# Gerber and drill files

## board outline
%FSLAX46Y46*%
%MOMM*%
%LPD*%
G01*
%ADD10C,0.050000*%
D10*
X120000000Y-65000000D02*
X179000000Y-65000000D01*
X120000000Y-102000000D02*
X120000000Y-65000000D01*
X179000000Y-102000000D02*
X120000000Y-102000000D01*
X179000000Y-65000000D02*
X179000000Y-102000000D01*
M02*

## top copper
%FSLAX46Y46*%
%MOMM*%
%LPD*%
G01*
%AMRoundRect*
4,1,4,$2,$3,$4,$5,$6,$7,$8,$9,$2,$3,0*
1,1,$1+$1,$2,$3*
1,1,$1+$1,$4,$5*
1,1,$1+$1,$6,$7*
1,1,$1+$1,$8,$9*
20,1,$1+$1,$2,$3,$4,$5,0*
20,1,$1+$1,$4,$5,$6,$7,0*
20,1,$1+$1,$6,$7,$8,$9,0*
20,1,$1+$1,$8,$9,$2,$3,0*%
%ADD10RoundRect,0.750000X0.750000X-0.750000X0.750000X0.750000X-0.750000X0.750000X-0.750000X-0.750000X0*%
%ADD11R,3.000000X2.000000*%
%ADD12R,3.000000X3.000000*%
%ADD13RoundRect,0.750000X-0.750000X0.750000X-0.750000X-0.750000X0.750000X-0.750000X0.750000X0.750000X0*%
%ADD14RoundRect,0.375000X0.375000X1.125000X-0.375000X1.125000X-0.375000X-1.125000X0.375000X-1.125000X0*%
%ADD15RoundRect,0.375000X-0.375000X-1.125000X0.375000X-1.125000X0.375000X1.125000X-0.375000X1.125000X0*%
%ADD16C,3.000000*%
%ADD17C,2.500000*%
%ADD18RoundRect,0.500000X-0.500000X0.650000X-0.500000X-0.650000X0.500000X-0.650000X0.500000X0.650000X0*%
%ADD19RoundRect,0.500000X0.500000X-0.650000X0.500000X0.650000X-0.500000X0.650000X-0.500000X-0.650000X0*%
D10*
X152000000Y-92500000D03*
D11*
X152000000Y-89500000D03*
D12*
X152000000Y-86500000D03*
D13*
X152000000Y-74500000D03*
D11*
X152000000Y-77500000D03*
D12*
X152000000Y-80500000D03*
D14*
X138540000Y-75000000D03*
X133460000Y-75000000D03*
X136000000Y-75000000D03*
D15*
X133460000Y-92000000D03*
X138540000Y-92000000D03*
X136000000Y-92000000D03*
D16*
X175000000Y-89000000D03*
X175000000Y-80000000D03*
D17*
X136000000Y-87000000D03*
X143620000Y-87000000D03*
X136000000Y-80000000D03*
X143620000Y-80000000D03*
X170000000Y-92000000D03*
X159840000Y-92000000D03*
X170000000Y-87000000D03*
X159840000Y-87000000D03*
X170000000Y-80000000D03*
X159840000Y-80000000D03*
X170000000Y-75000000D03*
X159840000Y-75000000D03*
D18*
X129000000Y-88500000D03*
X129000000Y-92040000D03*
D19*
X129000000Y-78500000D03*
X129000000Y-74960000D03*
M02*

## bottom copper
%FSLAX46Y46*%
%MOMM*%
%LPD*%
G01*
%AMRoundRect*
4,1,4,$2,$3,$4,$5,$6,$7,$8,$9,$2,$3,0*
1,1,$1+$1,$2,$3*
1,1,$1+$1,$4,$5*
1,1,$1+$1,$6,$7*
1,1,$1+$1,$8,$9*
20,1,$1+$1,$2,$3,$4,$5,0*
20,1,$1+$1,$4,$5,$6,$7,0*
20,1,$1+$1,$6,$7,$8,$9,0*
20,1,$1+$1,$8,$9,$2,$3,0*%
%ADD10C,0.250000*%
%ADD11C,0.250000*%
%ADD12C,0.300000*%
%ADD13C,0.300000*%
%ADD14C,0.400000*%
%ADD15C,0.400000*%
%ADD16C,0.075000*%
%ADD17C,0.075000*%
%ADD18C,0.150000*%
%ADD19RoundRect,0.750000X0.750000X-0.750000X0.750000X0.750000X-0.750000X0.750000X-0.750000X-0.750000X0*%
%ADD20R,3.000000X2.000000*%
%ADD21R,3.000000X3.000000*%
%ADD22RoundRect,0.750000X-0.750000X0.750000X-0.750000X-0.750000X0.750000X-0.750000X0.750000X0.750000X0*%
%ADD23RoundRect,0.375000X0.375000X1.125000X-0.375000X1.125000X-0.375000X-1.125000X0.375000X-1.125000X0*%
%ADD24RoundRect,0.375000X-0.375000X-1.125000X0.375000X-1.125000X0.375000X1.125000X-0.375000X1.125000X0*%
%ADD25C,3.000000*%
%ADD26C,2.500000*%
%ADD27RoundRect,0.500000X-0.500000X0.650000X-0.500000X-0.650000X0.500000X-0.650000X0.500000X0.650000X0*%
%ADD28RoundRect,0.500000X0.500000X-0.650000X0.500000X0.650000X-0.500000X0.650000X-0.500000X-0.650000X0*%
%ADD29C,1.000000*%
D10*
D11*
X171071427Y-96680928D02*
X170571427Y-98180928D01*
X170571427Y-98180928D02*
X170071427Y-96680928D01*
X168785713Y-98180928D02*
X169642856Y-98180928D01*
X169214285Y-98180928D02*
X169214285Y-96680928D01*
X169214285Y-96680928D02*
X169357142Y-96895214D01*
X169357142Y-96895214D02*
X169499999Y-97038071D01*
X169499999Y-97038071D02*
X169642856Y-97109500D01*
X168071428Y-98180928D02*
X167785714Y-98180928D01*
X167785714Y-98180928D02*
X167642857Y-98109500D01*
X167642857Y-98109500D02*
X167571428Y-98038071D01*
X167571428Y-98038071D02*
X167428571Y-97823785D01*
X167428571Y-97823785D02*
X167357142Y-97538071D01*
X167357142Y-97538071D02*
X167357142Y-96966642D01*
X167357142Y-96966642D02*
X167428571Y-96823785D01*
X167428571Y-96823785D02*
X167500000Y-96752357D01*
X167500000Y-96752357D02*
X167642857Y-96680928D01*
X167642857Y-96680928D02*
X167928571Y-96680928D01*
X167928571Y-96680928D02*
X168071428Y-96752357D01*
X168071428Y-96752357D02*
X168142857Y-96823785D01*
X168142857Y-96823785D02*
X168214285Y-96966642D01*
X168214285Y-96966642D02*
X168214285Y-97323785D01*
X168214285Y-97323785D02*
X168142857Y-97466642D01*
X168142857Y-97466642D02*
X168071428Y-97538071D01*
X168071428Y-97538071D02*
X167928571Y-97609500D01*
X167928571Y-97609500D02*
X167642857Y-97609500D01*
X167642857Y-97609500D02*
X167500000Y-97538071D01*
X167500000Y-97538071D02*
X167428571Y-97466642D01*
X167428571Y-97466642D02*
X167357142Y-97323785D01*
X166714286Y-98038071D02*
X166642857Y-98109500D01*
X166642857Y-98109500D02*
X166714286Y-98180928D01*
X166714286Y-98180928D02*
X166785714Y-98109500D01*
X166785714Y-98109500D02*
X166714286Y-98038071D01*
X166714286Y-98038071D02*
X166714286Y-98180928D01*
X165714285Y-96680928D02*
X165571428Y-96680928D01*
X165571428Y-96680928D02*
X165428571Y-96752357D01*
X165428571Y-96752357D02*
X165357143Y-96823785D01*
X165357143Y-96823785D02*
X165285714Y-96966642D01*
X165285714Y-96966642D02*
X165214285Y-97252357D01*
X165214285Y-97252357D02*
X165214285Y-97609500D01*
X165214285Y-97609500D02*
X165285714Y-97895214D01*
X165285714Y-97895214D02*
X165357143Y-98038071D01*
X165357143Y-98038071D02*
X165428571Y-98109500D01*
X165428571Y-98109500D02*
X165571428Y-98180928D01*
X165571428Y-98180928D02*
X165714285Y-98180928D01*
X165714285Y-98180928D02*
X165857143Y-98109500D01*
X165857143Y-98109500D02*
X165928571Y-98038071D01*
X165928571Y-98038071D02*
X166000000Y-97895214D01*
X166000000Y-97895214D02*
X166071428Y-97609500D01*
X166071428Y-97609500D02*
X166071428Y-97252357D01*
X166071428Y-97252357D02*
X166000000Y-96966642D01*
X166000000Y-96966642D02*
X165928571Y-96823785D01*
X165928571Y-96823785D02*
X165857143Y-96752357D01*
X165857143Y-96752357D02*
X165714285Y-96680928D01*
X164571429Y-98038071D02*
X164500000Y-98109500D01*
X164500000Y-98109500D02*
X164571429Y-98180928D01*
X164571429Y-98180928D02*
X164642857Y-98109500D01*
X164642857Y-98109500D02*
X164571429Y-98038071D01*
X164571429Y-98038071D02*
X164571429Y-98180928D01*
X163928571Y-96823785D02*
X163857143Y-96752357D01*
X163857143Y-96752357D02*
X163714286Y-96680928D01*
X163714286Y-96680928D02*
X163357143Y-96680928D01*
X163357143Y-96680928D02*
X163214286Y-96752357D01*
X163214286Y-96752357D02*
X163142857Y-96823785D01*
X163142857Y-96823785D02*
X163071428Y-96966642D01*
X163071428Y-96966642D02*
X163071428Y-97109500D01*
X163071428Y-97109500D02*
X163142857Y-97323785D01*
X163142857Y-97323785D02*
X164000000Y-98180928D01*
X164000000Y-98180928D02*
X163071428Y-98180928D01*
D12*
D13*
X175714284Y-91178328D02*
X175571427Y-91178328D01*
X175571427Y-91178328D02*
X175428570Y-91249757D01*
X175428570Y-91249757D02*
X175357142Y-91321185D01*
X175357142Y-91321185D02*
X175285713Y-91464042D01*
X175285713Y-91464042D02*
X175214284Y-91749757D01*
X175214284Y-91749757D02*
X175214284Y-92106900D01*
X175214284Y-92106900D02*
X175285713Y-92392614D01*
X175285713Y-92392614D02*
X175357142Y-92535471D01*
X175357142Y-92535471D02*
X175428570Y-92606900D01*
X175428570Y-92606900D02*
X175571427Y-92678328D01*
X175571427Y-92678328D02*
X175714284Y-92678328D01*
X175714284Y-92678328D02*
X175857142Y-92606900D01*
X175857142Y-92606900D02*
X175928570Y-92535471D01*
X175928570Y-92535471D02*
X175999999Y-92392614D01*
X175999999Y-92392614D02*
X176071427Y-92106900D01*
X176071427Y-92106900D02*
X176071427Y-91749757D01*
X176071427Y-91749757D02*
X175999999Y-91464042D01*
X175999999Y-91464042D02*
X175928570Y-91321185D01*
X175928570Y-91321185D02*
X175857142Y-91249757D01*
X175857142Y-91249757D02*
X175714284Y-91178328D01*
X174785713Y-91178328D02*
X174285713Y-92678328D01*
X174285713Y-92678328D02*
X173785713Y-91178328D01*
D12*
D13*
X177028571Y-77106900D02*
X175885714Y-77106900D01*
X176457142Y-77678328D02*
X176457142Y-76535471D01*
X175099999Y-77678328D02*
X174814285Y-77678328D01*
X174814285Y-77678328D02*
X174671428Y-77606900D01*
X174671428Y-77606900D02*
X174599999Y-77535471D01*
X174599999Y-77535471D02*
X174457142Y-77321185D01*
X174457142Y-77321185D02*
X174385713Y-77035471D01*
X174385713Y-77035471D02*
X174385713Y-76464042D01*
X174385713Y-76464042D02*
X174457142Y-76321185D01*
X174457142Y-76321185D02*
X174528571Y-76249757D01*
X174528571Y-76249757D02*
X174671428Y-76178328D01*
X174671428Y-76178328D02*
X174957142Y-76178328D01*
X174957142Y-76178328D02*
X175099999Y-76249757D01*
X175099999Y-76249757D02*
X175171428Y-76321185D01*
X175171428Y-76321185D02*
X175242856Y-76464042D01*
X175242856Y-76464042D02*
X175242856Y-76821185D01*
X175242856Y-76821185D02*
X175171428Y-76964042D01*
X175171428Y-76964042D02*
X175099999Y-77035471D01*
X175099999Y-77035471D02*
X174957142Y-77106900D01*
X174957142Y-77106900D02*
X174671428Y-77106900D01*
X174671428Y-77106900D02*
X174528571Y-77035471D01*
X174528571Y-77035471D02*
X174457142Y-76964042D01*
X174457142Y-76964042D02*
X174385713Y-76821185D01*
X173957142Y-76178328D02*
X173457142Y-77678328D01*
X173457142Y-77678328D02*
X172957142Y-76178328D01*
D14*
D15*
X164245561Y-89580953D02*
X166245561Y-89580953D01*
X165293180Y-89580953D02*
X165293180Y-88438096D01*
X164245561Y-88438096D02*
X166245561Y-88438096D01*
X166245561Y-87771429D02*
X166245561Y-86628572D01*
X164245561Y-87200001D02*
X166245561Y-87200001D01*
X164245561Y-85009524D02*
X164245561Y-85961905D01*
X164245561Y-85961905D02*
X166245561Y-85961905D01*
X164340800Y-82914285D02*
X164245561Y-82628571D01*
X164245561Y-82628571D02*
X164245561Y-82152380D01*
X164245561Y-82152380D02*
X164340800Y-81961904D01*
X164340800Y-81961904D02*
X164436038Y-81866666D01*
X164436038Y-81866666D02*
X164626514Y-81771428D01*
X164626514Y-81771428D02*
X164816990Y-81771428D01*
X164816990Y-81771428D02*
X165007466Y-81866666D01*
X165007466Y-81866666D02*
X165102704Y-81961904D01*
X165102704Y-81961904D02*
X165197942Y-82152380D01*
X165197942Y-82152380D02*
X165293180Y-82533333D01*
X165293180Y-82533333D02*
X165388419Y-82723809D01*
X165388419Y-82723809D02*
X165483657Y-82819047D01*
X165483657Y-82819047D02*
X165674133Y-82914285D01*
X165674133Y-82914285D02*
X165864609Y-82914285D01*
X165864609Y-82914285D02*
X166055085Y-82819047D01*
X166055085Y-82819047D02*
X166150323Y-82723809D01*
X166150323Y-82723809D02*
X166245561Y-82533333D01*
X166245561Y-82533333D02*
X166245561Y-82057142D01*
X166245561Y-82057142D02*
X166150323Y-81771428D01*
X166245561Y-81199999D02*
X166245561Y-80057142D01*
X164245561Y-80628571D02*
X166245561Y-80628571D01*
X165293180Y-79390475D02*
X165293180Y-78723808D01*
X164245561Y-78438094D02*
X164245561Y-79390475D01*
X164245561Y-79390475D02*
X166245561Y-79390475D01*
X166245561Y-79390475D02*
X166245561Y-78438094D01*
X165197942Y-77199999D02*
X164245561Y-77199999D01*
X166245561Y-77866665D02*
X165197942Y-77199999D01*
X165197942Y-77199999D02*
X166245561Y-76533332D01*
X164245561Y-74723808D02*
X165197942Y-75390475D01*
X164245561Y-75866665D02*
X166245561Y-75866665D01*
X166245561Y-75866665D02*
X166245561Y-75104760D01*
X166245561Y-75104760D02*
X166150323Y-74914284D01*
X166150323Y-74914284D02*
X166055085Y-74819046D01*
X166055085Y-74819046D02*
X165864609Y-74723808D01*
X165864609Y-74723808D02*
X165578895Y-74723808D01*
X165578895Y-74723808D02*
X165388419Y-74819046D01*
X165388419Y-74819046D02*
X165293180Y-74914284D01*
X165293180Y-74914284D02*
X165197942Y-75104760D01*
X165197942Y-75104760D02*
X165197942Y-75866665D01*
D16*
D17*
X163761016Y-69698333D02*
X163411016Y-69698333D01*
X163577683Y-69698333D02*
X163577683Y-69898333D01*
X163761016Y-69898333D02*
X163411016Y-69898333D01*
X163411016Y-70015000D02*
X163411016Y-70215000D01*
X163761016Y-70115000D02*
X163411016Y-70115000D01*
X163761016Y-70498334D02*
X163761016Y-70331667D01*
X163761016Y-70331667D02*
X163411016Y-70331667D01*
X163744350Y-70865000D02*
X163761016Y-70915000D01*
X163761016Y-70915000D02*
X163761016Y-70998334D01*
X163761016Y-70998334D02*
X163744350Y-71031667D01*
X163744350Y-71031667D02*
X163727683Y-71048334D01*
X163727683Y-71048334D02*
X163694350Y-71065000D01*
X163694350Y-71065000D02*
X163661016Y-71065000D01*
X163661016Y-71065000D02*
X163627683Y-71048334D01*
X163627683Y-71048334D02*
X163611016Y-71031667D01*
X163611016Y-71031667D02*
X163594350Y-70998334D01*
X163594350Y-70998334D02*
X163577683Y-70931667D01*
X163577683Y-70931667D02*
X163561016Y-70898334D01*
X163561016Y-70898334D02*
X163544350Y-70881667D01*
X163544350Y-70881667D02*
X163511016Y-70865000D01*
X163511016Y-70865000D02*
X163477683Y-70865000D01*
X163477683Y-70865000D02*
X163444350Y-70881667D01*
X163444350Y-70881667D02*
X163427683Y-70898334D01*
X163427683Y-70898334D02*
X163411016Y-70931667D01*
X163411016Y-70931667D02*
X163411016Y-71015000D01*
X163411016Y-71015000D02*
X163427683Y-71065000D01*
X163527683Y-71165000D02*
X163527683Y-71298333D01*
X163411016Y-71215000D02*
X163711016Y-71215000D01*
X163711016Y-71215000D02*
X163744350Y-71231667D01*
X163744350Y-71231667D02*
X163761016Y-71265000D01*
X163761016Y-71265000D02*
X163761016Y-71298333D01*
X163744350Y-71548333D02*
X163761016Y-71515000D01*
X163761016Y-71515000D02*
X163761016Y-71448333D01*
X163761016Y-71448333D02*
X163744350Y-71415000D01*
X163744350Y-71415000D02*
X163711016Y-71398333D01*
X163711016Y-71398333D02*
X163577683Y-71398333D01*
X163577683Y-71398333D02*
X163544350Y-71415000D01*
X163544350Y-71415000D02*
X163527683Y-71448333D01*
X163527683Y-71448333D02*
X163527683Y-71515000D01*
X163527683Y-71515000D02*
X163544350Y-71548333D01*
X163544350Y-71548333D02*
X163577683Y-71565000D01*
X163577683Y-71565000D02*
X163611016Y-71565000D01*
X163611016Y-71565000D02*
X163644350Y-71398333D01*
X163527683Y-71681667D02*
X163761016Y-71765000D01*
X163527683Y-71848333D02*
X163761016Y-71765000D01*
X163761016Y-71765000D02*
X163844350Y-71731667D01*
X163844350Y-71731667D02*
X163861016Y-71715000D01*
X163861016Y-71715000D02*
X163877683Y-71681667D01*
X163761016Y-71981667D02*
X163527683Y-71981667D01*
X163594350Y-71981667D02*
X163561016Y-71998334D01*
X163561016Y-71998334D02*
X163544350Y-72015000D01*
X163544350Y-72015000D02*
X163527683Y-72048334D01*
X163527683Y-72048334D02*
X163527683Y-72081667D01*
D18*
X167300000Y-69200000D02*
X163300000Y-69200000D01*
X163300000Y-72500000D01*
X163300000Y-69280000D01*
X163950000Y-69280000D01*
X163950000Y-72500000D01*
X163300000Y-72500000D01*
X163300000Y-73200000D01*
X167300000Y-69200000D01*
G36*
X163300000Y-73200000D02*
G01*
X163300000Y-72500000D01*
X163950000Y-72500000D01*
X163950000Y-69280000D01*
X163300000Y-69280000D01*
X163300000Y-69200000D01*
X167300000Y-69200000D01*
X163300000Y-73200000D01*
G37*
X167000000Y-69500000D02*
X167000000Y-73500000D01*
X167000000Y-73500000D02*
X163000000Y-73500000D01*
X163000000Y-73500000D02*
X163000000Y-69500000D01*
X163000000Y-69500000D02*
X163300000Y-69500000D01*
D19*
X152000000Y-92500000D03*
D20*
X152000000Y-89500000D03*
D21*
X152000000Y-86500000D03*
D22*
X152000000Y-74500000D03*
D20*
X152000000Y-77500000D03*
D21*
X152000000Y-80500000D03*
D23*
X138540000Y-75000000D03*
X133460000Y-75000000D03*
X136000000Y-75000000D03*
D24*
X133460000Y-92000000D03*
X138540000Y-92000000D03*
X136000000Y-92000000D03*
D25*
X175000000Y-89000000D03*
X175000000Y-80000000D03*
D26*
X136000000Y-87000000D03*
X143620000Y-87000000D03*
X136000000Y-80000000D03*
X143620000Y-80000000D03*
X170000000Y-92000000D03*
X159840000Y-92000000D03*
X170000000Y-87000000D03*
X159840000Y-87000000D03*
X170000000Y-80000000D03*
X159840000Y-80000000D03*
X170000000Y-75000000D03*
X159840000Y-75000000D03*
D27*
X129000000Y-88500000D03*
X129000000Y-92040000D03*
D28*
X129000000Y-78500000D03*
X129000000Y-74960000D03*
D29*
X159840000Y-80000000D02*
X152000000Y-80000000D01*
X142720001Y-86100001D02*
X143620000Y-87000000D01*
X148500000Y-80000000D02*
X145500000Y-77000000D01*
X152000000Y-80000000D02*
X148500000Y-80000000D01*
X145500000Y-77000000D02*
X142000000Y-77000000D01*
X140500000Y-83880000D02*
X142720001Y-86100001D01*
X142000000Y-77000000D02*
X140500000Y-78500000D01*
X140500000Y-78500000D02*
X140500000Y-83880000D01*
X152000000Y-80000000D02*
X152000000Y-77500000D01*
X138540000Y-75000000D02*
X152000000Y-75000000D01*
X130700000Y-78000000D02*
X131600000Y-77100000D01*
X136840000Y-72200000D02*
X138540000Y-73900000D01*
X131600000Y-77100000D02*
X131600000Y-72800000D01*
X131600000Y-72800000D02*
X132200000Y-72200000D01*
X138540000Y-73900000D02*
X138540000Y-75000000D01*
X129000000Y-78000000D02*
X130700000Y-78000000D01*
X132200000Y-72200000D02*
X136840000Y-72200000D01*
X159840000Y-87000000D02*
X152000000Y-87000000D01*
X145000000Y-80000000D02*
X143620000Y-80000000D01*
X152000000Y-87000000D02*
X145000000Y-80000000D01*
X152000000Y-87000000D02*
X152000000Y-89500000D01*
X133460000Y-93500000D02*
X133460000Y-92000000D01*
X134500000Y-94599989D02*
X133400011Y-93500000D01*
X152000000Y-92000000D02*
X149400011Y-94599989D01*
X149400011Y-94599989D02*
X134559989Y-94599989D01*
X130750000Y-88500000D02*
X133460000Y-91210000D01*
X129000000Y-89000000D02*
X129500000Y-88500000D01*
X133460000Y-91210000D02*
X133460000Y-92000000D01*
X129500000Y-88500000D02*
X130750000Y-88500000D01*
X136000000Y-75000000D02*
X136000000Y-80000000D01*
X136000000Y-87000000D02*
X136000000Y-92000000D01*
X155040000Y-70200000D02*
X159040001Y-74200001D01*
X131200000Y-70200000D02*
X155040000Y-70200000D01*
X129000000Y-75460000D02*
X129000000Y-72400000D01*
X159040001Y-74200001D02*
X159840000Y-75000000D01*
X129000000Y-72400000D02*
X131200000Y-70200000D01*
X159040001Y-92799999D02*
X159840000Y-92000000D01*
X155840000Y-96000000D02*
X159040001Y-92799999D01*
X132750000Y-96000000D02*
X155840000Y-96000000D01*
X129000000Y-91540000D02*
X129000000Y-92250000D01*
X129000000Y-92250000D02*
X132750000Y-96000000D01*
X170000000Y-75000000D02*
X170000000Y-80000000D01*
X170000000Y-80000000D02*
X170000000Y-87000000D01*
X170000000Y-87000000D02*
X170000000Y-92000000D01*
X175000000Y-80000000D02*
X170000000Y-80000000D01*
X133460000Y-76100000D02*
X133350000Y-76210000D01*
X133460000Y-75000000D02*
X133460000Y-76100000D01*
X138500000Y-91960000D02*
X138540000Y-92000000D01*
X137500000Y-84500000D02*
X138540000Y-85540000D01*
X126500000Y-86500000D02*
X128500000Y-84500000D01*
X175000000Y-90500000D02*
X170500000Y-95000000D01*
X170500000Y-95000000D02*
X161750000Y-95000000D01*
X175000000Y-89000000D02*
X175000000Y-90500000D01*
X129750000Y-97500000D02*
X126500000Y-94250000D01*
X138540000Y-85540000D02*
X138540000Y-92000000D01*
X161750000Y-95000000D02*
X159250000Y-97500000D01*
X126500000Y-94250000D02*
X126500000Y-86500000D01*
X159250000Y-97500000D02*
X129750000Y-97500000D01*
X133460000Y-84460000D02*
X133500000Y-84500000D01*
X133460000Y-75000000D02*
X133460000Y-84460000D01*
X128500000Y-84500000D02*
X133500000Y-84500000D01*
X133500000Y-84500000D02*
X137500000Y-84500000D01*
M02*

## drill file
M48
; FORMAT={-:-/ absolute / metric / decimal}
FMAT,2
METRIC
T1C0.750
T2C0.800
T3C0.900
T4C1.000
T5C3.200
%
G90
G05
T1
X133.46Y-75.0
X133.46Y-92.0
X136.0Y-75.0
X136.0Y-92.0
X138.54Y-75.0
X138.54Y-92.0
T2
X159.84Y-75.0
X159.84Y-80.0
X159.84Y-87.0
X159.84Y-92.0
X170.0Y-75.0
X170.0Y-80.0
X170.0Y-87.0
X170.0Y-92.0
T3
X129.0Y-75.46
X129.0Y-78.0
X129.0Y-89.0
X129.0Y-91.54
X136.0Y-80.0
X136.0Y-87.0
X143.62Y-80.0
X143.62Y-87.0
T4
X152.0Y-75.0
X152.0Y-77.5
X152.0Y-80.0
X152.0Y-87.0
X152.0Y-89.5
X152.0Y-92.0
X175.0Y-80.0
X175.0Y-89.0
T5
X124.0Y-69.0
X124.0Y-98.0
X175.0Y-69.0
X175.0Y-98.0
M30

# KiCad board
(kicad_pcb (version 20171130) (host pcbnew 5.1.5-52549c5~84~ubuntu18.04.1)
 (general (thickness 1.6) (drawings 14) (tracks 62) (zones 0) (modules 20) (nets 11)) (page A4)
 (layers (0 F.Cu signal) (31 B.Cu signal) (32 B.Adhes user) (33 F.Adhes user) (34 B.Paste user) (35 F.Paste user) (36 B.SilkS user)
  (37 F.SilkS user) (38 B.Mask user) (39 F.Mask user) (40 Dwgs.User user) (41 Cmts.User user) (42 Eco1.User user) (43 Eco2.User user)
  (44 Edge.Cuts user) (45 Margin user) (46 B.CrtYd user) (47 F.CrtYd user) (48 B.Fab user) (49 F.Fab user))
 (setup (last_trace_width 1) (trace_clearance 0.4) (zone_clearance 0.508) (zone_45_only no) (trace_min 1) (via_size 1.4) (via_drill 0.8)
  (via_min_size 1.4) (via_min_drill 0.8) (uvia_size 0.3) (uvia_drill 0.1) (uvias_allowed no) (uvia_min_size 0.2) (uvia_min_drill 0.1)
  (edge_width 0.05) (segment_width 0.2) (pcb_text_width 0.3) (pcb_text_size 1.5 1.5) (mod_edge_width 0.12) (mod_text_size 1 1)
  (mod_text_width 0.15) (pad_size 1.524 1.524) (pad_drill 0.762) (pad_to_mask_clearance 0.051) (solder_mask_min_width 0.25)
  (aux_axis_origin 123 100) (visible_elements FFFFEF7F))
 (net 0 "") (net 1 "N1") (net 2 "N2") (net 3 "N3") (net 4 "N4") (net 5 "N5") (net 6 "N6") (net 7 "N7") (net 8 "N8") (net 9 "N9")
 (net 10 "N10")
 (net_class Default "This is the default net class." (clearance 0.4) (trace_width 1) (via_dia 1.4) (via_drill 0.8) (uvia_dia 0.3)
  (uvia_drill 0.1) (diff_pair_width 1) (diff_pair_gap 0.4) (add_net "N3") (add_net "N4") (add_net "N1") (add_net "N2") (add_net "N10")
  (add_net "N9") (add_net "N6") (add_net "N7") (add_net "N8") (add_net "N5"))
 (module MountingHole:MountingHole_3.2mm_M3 (layer F.Cu) (at 124 98)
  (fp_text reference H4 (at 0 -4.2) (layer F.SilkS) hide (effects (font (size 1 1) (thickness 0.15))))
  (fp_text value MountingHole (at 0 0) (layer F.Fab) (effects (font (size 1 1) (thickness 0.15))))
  (pad 1 np_thru_hole circle (at 0 0) (size 3.2 3.2) (drill 3.2) (layers *.Cu *.Mask)))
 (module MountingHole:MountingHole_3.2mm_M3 (layer F.Cu) (at 124 69)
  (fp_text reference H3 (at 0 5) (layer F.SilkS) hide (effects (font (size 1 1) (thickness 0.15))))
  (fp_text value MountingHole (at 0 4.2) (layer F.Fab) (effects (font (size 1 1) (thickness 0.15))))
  (pad 1 np_thru_hole circle (at 0 0) (size 3.2 3.2) (drill 3.2) (layers *.Cu *.Mask)))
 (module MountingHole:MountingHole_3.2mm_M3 (layer F.Cu) (at 175 98)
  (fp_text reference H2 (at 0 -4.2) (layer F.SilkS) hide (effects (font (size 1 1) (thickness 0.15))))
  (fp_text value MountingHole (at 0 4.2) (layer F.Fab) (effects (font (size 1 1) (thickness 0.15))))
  (pad 1 np_thru_hole circle (at 0 0) (size 3.2 3.2) (drill 3.2) (layers *.Cu *.Mask)))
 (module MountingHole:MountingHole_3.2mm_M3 (layer F.Cu) (at 175 69)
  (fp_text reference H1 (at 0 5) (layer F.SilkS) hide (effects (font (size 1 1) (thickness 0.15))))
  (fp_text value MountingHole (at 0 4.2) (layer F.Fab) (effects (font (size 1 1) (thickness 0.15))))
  (pad 1 np_thru_hole circle (at 0 0) (size 3.2 3.2) (drill 3.2) (layers *.Cu *.Mask)))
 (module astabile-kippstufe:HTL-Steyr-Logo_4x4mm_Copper (layer B.Cu) (at 165 71.5 90)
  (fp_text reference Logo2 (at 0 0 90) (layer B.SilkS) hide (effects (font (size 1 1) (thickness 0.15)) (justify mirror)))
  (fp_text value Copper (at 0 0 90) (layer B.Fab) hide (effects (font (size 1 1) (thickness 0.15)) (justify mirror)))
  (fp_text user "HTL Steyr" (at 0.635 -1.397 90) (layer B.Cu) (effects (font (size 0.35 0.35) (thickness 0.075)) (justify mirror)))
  (fp_poly
   (pts (xy 2.3 2.3) (xy 2.3 -1.7) (xy -1 -1.7) (xy 2.22 -1.7) (xy 2.22 -1.05) (xy -1 -1.05) (xy -1 -1.7) (xy -1.7 -1.7)) (layer B.Cu)
   (width 0.15))
  (fp_line (start 2 2) (end -2 2) (layer B.Cu) (width 0.15)) (fp_line (start -2 2) (end -2 -2) (layer B.Cu) (width 0.15))
  (fp_line (start -2 -2) (end 2 -2) (layer B.Cu) (width 0.15))
  (fp_line (start 2 -2) (end 2 -1.7) (layer B.Cu) (width 0.15)))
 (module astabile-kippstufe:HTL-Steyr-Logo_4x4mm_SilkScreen (layer F.Cu) (at 162 98)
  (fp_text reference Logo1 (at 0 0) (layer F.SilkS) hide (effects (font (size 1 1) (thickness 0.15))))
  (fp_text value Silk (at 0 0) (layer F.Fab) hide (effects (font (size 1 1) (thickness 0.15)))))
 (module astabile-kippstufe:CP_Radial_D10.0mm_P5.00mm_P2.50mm (layer F.Cu) (at 152 92 90)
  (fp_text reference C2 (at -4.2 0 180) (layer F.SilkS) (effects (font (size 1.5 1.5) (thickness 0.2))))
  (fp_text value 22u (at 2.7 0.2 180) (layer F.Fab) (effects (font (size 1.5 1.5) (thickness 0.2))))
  (pad 1 thru_hole roundrect (at 0 0 90) (size 3 3) (drill 1 (offset -0.5 0)) (layers *.Cu *.Mask) (roundrect_rratio 0.25) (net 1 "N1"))
  (pad 2 thru_hole rect (at 2.5 0 90) (size 2 3) (drill 1) (layers *.Cu *.Mask) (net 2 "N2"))
  (pad 2 thru_hole rect (at 5 0 90) (size 3 3) (drill 1 (offset 0.5 0)) (layers *.Cu *.Mask) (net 2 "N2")))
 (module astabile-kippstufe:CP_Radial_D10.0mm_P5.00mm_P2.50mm (layer F.Cu) (at 152 75 270)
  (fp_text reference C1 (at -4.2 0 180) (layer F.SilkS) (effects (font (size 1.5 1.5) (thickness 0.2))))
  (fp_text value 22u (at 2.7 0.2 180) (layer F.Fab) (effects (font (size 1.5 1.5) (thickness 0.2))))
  (pad 1 thru_hole roundrect (at 0 0 270) (size 3 3) (drill 1 (offset -0.5 0)) (layers *.Cu *.Mask) (roundrect_rratio 0.25) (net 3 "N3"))
  (pad 2 thru_hole rect (at 2.5 0 270) (size 2 3) (drill 1) (layers *.Cu *.Mask) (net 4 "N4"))
  (pad 2 thru_hole rect (at 5 0 270) (size 3 3) (drill 1 (offset 0.5 0)) (layers *.Cu *.Mask) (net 4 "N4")))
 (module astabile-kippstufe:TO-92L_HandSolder (layer F.Cu) (at 138.54 75 180)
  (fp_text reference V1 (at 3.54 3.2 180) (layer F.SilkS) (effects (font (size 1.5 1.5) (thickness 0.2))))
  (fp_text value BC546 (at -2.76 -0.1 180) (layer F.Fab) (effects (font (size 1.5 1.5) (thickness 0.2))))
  (pad 1 thru_hole roundrect (at 0 0 180) (size 1.5 3) (drill 0.75) (layers *.Cu *.Mask) (roundrect_rratio 0.25) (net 3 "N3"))
  (pad 3 thru_hole roundrect (at 5.08 0 180) (size 1.5 3) (drill 0.75) (layers *.Cu *.Mask) (roundrect_rratio 0.25) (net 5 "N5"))
  (pad 2 thru_hole roundrect (at 2.54 0 180) (size 1.5 3) (drill 0.75) (layers *.Cu *.Mask) (roundrect_rratio 0.25) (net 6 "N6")))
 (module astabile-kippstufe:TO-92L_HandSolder (layer F.Cu) (at 133.46 92)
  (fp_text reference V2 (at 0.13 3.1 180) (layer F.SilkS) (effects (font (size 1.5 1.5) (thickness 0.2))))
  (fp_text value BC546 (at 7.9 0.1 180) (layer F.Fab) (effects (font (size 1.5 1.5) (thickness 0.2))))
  (pad 1 thru_hole roundrect (at 0 0) (size 1.5 3) (drill 0.75) (layers *.Cu *.Mask) (roundrect_rratio 0.25) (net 1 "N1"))
  (pad 3 thru_hole roundrect (at 5.08 0) (size 1.5 3) (drill 0.75) (layers *.Cu *.Mask) (roundrect_rratio 0.25) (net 5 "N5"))
  (pad 2 thru_hole roundrect (at 2.54 0) (size 1.5 3) (drill 0.75) (layers *.Cu *.Mask) (roundrect_rratio 0.25) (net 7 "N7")))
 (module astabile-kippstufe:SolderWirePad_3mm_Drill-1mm (layer F.Cu) (at 175 89)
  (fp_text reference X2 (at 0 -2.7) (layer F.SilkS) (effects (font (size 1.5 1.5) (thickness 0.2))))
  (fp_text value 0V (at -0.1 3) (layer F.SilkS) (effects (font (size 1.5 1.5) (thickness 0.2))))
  (pad 1 thru_hole circle (at 0 0) (size 3 3) (drill 1) (layers *.Cu *.Mask) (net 5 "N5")))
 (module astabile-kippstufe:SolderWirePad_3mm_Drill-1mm (layer F.Cu) (at 175 80)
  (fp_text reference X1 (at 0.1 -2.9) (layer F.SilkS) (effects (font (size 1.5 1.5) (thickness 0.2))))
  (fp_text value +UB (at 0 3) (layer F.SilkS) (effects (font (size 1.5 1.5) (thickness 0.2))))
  (pad 1 thru_hole circle (at 0 0) (size 3 3) (drill 1) (layers *.Cu *.Mask) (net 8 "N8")))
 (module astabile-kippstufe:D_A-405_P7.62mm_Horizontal (layer F.Cu) (at 136 87)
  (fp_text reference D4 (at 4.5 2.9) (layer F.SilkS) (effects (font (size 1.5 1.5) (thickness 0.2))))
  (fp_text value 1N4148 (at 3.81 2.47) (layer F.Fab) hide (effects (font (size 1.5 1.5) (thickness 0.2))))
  (pad 1 thru_hole circle (at 0 0) (size 2.5 2.5) (drill 0.9) (layers *.Cu *.Mask) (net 7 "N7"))
  (pad 2 thru_hole circle (at 7.62 0) (size 2.5 2.5) (drill 0.9) (layers *.Cu *.Mask) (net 4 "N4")))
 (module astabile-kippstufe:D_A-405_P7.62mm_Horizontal (layer F.Cu) (at 136 80)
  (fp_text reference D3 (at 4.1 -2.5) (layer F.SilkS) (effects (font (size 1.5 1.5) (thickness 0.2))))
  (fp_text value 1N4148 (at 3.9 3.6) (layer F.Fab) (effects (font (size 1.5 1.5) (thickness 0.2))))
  (pad 1 thru_hole circle (at 0 0) (size 2.5 2.5) (drill 0.9) (layers *.Cu *.Mask) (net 6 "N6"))
  (pad 2 thru_hole circle (at 7.62 0) (size 2.5 2.5) (drill 0.9) (layers *.Cu *.Mask) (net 2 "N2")))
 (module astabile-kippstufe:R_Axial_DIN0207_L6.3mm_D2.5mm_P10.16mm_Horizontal (layer F.Cu) (at 170 92 180)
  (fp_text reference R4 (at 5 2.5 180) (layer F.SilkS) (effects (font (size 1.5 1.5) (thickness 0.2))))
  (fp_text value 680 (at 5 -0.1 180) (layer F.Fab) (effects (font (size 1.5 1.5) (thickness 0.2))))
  (pad 1 thru_hole circle (at 0 0 180) (size 2.5 2.5) (drill 0.8) (layers *.Cu *.Mask) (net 8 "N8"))
  (pad 2 thru_hole circle (at 10.16 0 180) (size 2.5 2.5) (drill 0.8) (layers *.Cu *.Mask) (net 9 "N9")))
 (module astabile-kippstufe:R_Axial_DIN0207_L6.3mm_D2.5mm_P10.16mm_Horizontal (layer F.Cu) (at 170 87 180)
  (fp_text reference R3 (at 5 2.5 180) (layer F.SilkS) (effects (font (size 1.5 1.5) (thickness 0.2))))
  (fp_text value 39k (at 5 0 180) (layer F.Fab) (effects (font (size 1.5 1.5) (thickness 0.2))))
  (pad 1 thru_hole circle (at 0 0 180) (size 2.5 2.5) (drill 0.8) (layers *.Cu *.Mask) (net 8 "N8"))
  (pad 2 thru_hole circle (at 10.16 0 180) (size 2.5 2.5) (drill 0.8) (layers *.Cu *.Mask) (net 2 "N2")))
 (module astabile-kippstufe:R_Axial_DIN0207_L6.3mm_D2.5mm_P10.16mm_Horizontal (layer F.Cu) (at 170 80 180)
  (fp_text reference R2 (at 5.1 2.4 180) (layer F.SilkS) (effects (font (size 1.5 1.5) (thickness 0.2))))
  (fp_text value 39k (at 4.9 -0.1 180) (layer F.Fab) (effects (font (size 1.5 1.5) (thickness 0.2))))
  (pad 1 thru_hole circle (at 0 0 180) (size 2.5 2.5) (drill 0.8) (layers *.Cu *.Mask) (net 8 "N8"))
  (pad 2 thru_hole circle (at 10.16 0 180) (size 2.5 2.5) (drill 0.8) (layers *.Cu *.Mask) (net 4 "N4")))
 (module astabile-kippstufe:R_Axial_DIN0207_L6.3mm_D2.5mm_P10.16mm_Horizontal (layer F.Cu) (at 170 75 180)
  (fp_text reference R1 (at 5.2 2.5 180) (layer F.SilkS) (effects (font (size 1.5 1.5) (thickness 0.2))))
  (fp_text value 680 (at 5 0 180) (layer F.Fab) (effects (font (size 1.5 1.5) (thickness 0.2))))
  (pad 1 thru_hole circle (at 0 0 180) (size 2.5 2.5) (drill 0.8) (layers *.Cu *.Mask) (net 8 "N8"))
  (pad 2 thru_hole circle (at 10.16 0 180) (size 2.5 2.5) (drill 0.8) (layers *.Cu *.Mask) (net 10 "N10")))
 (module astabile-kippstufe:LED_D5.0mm (layer F.Cu) (at 129 89 270)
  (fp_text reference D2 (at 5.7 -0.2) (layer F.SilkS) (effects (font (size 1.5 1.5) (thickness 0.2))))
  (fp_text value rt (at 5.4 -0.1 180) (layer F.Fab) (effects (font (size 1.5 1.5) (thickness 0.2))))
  (pad 1 thru_hole roundrect (at 0 0 270) (size 2.3 2) (drill 0.9 (offset -0.5 0)) (layers *.Cu *.Mask) (roundrect_rratio 0.25) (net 1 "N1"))
  (pad 2 thru_hole roundrect (at 2.54 0 270) (size 2.3 2) (drill 0.9 (offset 0.5 0)) (layers *.Cu *.Mask) (roundrect_rratio 0.25)
   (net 9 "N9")))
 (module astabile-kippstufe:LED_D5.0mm (layer F.Cu) (at 129 78 90)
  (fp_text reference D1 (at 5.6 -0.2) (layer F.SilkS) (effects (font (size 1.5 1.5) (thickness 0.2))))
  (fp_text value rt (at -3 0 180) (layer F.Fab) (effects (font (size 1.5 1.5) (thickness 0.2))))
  (pad 1 thru_hole roundrect (at 0 0 90) (size 2.3 2) (drill 0.9 (offset -0.5 0)) (layers *.Cu *.Mask) (roundrect_rratio 0.25) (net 3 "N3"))
  (pad 2 thru_hole roundrect (at 2.54 0 90) (size 2.3 2) (drill 0.9 (offset 0.5 0)) (layers *.Cu *.Mask) (roundrect_rratio 0.25)
   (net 10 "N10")))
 (gr_line (start 120 65) (end 179 65) (layer Edge.Cuts) (width 0.05))
 (gr_line (start 120 102) (end 120 65) (layer Edge.Cuts) (width 0.05))
 (gr_line (start 179 102) (end 120 102) (layer Edge.Cuts) (width 0.05))
 (gr_line (start 179 65) (end 179 102) (layer Edge.Cuts) (width 0.05))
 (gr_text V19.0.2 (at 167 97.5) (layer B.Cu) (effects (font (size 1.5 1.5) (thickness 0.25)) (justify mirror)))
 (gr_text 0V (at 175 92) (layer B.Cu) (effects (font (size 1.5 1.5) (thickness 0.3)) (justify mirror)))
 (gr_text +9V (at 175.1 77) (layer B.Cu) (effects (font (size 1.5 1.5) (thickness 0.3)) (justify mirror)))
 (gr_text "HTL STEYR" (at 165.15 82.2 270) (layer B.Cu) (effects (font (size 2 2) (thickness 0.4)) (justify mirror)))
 (segment (start 159.84 80) (end 152 80) (width 1) (layer B.Cu) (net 4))
 (segment (start 142.720001 86.100001) (end 143.62 87) (width 1) (layer B.Cu) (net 4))
 (segment (start 148.5 80) (end 145.5 77) (width 1) (layer B.Cu) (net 4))
 (segment (start 152 80) (end 148.5 80) (width 1) (layer B.Cu) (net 4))
 (segment (start 145.5 77) (end 142 77) (width 1) (layer B.Cu) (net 4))
 (segment (start 140.5 83.88) (end 142.720001 86.100001) (width 1) (layer B.Cu) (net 4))
 (segment (start 142 77) (end 140.5 78.5) (width 1) (layer B.Cu) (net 4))
 (segment (start 140.5 78.5) (end 140.5 83.88) (width 1) (layer B.Cu) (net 4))
 (segment (start 152 80) (end 152 77.5) (width 1) (layer B.Cu) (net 4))
 (segment (start 138.54 75) (end 152 75) (width 1) (layer B.Cu) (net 3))
 (segment (start 130.7 78) (end 131.6 77.1) (width 1) (layer B.Cu) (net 3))
 (segment (start 136.84 72.2) (end 138.54 73.9) (width 1) (layer B.Cu) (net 3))
 (segment (start 131.6 77.1) (end 131.6 72.8) (width 1) (layer B.Cu) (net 3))
 (segment (start 131.6 72.8) (end 132.2 72.2) (width 1) (layer B.Cu) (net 3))
 (segment (start 138.54 73.9) (end 138.54 75) (width 1) (layer B.Cu) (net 3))
 (segment (start 129 78) (end 130.7 78) (width 1) (layer B.Cu) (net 3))
 (segment (start 132.2 72.2) (end 136.84 72.2) (width 1) (layer B.Cu) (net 3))
 (segment (start 159.84 87) (end 152 87) (width 1) (layer B.Cu) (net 2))
 (segment (start 145 80) (end 143.62 80) (width 1) (layer B.Cu) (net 2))
 (segment (start 152 87) (end 145 80) (width 1) (layer B.Cu) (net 2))
 (segment (start 152 87) (end 152 89.5) (width 1) (layer B.Cu) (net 2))
 (segment (start 133.46 93.5) (end 133.46 92) (width 1) (layer B.Cu) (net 1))
 (segment (start 134.5 94.599989) (end 133.400011 93.5) (width 1) (layer B.Cu) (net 1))
 (segment (start 152 92) (end 149.400011 94.599989) (width 1) (layer B.Cu) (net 1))
 (segment (start 149.400011 94.599989) (end 134.559989 94.599989) (width 1) (layer B.Cu) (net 1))
 (segment (start 130.75 88.5) (end 133.46 91.21) (width 1) (layer B.Cu) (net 1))
 (segment (start 129 89) (end 129.5 88.5) (width 1) (layer B.Cu) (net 1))
 (segment (start 133.46 91.21) (end 133.46 92) (width 1) (layer B.Cu) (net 1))
 (segment (start 129.5 88.5) (end 130.75 88.5) (width 1) (layer B.Cu) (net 1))
 (segment (start 136 75) (end 136 80) (width 1) (layer B.Cu) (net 6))
 (segment (start 136 87) (end 136 92) (width 1) (layer B.Cu) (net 7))
 (segment (start 155.04 70.2) (end 159.040001 74.200001) (width 1) (layer B.Cu) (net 10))
 (segment (start 131.2 70.2) (end 155.04 70.2) (width 1) (layer B.Cu) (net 10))
 (segment (start 129 75.46) (end 129 72.4) (width 1) (layer B.Cu) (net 10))
 (segment (start 159.040001 74.200001) (end 159.84 75) (width 1) (layer B.Cu) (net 10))
 (segment (start 129 72.4) (end 131.2 70.2) (width 1) (layer B.Cu) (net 10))
 (segment (start 159.040001 92.799999) (end 159.84 92) (width 1) (layer B.Cu) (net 9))
 (segment (start 155.84 96) (end 159.040001 92.799999) (width 1) (layer B.Cu) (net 9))
 (segment (start 132.75 96) (end 155.84 96) (width 1) (layer B.Cu) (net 9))
 (segment (start 129 91.54) (end 129 92.25) (width 1) (layer B.Cu) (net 9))
 (segment (start 129 92.25) (end 132.75 96) (width 1) (layer B.Cu) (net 9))
 (segment (start 170 75) (end 170 80) (width 1) (layer B.Cu) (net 8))
 (segment (start 170 80) (end 170 87) (width 1) (layer B.Cu) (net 8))
 (segment (start 170 87) (end 170 92) (width 1) (layer B.Cu) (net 8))
 (segment (start 175 80) (end 170 80) (width 1) (layer B.Cu) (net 8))
 (segment (start 133.46 76.1) (end 133.35 76.21) (width 1) (layer B.Cu) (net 5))
 (segment (start 133.46 75) (end 133.46 76.1) (width 1) (layer B.Cu) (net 5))
 (segment (start 138.5 91.96) (end 138.54 92) (width 1) (layer B.Cu) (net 5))
 (segment (start 137.5 84.5) (end 138.54 85.54) (width 1) (layer B.Cu) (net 5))
 (segment (start 126.5 86.5) (end 128.5 84.5) (width 1) (layer B.Cu) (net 5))
 (segment (start 175 90.5) (end 170.5 95) (width 1) (layer B.Cu) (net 5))
 (segment (start 170.5 95) (end 161.75 95) (width 1) (layer B.Cu) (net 5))
 (segment (start 175 89) (end 175 90.5) (width 1) (layer B.Cu) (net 5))
 (segment (start 129.75 97.5) (end 126.5 94.25) (width 1) (layer B.Cu) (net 5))
 (segment (start 138.54 85.54) (end 138.54 92) (width 1) (layer B.Cu) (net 5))
 (segment (start 161.75 95) (end 159.25 97.5) (width 1) (layer B.Cu) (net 5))
 (segment (start 126.5 94.25) (end 126.5 86.5) (width 1) (layer B.Cu) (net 5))
 (segment (start 159.25 97.5) (end 129.75 97.5) (width 1) (layer B.Cu) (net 5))
 (segment (start 133.46 84.46) (end 133.5 84.5) (width 1) (layer B.Cu) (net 5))
 (segment (start 133.46 75) (end 133.46 84.46) (width 1) (layer B.Cu) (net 5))
 (segment (start 128.5 84.5) (end 133.5 84.5) (width 1) (layer B.Cu) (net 5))
 (segment (start 133.5 84.5) (end 137.5 84.5) (width 1) (layer B.Cu) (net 5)))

